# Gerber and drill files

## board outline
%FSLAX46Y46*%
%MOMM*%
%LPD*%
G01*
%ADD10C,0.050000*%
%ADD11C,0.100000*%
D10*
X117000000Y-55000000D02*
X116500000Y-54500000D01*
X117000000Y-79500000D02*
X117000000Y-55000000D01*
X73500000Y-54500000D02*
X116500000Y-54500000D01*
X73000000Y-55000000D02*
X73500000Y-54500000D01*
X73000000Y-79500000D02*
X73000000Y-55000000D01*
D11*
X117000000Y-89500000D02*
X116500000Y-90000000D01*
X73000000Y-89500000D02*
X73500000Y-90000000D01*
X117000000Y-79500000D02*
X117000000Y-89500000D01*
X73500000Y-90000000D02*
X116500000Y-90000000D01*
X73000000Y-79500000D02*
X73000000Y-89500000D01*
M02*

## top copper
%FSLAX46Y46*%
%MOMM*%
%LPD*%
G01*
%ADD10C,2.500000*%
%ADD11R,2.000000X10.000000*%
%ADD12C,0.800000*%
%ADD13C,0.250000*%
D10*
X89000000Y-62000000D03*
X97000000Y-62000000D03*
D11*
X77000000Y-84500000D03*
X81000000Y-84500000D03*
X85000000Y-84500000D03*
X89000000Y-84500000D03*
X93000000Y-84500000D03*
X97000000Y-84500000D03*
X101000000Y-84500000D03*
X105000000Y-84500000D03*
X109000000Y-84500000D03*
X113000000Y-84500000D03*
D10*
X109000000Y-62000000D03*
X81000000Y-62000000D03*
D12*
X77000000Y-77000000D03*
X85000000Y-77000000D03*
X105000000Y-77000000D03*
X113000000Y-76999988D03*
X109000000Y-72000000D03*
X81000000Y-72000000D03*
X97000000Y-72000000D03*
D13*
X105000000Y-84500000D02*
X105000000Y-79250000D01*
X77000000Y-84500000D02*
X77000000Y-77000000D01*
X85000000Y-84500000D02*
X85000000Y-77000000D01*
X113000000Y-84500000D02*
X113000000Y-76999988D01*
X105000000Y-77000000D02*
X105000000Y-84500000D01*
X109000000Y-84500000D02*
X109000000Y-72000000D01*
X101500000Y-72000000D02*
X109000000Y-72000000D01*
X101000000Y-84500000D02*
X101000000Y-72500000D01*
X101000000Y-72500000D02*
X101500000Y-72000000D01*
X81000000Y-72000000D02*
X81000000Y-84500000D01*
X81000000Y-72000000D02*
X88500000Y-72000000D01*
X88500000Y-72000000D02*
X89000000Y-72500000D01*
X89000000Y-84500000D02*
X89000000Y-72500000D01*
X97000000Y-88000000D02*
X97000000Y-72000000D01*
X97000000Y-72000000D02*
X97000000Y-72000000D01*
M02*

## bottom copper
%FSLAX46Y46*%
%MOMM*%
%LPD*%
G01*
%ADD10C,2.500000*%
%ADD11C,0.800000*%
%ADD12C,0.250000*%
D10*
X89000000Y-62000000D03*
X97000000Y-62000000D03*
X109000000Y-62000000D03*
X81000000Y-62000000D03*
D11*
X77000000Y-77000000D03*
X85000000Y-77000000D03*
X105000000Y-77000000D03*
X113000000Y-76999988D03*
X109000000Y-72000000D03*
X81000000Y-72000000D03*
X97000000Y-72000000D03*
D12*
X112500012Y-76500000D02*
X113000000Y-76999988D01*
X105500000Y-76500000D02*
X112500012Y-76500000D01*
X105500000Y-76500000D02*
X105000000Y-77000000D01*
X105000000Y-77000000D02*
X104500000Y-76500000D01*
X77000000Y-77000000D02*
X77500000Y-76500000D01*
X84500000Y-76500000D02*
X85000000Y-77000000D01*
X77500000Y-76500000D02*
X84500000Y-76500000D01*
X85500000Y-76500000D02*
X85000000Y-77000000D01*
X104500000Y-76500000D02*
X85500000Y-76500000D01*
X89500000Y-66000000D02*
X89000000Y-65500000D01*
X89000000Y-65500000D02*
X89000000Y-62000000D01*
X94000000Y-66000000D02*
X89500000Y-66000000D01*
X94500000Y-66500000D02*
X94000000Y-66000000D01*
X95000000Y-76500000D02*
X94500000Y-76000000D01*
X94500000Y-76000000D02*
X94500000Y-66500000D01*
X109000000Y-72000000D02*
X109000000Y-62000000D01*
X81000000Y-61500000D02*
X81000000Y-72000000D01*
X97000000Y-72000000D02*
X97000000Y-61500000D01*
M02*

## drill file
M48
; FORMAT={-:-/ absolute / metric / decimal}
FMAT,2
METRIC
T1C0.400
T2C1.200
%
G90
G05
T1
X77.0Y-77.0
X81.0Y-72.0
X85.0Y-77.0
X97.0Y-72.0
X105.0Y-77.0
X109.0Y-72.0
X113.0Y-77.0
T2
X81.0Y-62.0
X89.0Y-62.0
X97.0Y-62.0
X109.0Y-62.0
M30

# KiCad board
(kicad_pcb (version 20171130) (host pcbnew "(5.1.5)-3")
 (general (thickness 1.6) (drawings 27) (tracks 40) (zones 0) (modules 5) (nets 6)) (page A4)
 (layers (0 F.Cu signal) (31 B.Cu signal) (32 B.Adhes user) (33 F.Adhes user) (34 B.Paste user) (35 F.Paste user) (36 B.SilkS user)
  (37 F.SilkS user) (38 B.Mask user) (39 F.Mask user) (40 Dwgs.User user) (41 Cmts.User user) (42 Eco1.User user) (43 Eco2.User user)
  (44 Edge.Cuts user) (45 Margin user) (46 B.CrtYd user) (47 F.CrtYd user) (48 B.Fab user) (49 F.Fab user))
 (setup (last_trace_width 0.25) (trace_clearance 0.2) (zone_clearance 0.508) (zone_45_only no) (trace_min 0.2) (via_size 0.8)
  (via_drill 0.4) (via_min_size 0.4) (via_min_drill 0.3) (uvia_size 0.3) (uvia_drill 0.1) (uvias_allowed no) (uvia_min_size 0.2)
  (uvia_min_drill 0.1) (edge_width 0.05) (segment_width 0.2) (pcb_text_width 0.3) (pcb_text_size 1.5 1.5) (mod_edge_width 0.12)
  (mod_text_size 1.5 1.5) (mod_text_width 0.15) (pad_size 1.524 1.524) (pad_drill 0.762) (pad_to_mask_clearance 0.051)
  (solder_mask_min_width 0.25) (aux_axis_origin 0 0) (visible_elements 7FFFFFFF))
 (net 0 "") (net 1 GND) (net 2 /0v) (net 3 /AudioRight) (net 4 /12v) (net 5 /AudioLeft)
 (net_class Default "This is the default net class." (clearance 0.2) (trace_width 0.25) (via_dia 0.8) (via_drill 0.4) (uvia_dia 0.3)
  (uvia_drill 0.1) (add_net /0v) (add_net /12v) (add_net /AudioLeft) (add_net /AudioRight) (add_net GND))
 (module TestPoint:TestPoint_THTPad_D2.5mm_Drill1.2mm (layer F.Cu) (at 89 62)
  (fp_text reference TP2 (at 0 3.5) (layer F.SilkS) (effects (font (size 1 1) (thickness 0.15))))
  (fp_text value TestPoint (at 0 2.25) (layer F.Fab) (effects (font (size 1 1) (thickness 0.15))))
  (pad 1 thru_hole circle (at 0 0) (size 2.5 2.5) (drill 1.2) (layers *.Cu *.Mask) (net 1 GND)))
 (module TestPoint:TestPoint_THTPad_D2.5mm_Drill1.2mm (layer F.Cu) (at 97 62)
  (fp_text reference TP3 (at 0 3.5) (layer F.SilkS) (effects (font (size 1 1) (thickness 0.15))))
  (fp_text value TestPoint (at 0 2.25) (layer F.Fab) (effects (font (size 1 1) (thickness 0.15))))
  (pad 1 thru_hole circle (at 0 0) (size 2.5 2.5) (drill 1.2) (layers *.Cu *.Mask) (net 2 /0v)))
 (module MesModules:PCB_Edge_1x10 (layer F.Cu) (at 77 89.5)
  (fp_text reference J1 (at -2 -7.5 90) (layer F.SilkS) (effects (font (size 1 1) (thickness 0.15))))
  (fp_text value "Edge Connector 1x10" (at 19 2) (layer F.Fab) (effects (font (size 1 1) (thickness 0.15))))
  (fp_line (start 40 0) (end 39.5 0.5) (layer Edge.Cuts) (width 0.1))
  (fp_line (start -4 0) (end -3.5 0.5) (layer Edge.Cuts) (width 0.1))
  (fp_line (start 40 -10) (end 40 0) (layer Edge.Cuts) (width 0.1))
  (fp_line (start -3.5 0.5) (end 39.5 0.5) (layer Edge.Cuts) (width 0.1))
  (fp_line (start -4 -10) (end -4 0) (layer Edge.Cuts) (width 0.1))
  (pad 10 connect rect (at 0 -5) (size 2 10) (layers F.Cu F.Mask) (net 1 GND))
  (pad 9 connect rect (at 4 -5) (size 2 10) (layers F.Cu F.Mask) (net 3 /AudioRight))
  (pad 8 connect rect (at 8 -5) (size 2 10) (layers F.Cu F.Mask) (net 1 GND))
  (pad 7 connect rect (at 12 -5) (size 2 10) (layers F.Cu F.Mask) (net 3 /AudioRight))
  (pad 6 connect rect (at 16 -5) (size 2 10) (layers F.Cu F.Mask) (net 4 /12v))
  (pad 5 connect rect (at 20 -5) (size 2 10) (layers F.Cu F.Mask) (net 2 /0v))
  (pad 4 connect rect (at 24 -5) (size 2 10) (layers F.Cu F.Mask) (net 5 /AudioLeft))
  (pad 3 connect rect (at 28 -5) (size 2 10) (layers F.Cu F.Mask) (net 1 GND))
  (pad 2 connect rect (at 32 -5) (size 2 10) (layers F.Cu F.Mask) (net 5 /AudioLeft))
  (pad 1 connect rect (at 36 -5) (size 2 10) (layers F.Cu F.Mask) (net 1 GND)))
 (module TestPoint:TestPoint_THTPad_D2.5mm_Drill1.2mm (layer F.Cu) (at 109 62)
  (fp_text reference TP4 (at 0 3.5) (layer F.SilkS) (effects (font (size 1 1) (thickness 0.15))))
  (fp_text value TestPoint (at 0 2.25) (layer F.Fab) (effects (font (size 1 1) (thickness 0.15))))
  (pad 1 thru_hole circle (at 0 0) (size 2.5 2.5) (drill 1.2) (layers *.Cu *.Mask) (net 5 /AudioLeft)))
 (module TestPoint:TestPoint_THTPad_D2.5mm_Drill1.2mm (layer F.Cu) (at 81 62)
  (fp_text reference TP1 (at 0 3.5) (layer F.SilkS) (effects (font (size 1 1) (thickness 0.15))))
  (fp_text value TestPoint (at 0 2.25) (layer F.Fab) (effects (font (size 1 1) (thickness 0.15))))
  (pad 1 thru_hole circle (at 0 0) (size 2.5 2.5) (drill 1.2) (layers *.Cu *.Mask) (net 3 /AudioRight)))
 (gr_line (start 117 55) (end 116.5 54.5) (layer Edge.Cuts) (width 0.05))
 (gr_line (start 117 79.5) (end 117 55) (layer Edge.Cuts) (width 0.05))
 (gr_line (start 73.5 54.5) (end 116.5 54.5) (layer Edge.Cuts) (width 0.05))
 (gr_line (start 73 55) (end 73.5 54.5) (layer Edge.Cuts) (width 0.05))
 (gr_line (start 73 79.5) (end 73 55) (layer Edge.Cuts) (width 0.05))
 (via (at 77 77) (size 0.8) (drill 0.4) (layers F.Cu B.Cu) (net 1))
 (via (at 85 77) (size 0.8) (drill 0.4) (layers F.Cu B.Cu) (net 1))
 (via (at 105 77) (size 0.8) (drill 0.4) (layers F.Cu B.Cu) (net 1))
 (via (at 113 76.999988) (size 0.8) (drill 0.4) (layers F.Cu B.Cu) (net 1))
 (segment (start 105 84.5) (end 105 79.25) (width 0.25) (layer F.Cu) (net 1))
 (segment (start 112.500012 76.5) (end 113 76.999988) (width 0.25) (layer B.Cu) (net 1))
 (segment (start 105.5 76.5) (end 112.500012 76.5) (width 0.25) (layer B.Cu) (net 1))
 (segment (start 105.5 76.5) (end 105 77) (width 0.25) (layer B.Cu) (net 1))
 (segment (start 105 77) (end 104.5 76.5) (width 0.25) (layer B.Cu) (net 1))
 (segment (start 77 77) (end 77.5 76.5) (width 0.25) (layer B.Cu) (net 1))
 (segment (start 77 84.5) (end 77 77) (width 0.25) (layer F.Cu) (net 1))
 (segment (start 85 84.5) (end 85 77) (width 0.25) (layer F.Cu) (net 1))
 (segment (start 113 84.5) (end 113 76.999988) (width 0.25) (layer F.Cu) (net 1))
 (segment (start 105 77) (end 105 84.5) (width 0.25) (layer F.Cu) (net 1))
 (segment (start 84.5 76.5) (end 85 77) (width 0.25) (layer B.Cu) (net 1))
 (segment (start 77.5 76.5) (end 84.5 76.5) (width 0.25) (layer B.Cu) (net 1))
 (segment (start 85.5 76.5) (end 85 77) (width 0.25) (layer B.Cu) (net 1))
 (segment (start 104.5 76.5) (end 85.5 76.5) (width 0.25) (layer B.Cu) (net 1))
 (segment (start 89.5 66) (end 89 65.5) (width 0.25) (layer B.Cu) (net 1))
 (segment (start 89 65.5) (end 89 62) (width 0.25) (layer B.Cu) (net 1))
 (segment (start 94 66) (end 89.5 66) (width 0.25) (layer B.Cu) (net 1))
 (segment (start 94.5 66.5) (end 94 66) (width 0.25) (layer B.Cu) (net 1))
 (segment (start 95 76.5) (end 94.5 76) (width 0.25) (layer B.Cu) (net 1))
 (segment (start 94.5 76) (end 94.5 66.5) (width 0.25) (layer B.Cu) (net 1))
 (via (at 109 72) (size 0.8) (drill 0.4) (layers F.Cu B.Cu) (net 5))
 (segment (start 109 84.5) (end 109 72) (width 0.25) (layer F.Cu) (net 5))
 (segment (start 101.5 72) (end 109 72) (width 0.25) (layer F.Cu) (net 5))
 (segment (start 101 84.5) (end 101 72.5) (width 0.25) (layer F.Cu) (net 5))
 (segment (start 101 72.5) (end 101.5 72) (width 0.25) (layer F.Cu) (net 5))
 (segment (start 109 72) (end 109 62) (width 0.25) (layer B.Cu) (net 5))
 (segment (start 81 72) (end 81 84.5) (width 0.25) (layer F.Cu) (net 3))
 (via (at 81 72) (size 0.8) (drill 0.4) (layers F.Cu B.Cu) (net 3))
 (segment (start 81 72) (end 88.5 72) (width 0.25) (layer F.Cu) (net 3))
 (segment (start 88.5 72) (end 89 72.5) (width 0.25) (layer F.Cu) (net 3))
 (segment (start 89 84.5) (end 89 72.5) (width 0.25) (layer F.Cu) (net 3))
 (segment (start 81 61.5) (end 81 72) (width 0.25) (layer B.Cu) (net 3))
 (segment (start 97 88) (end 97 72) (width 0.25) (layer F.Cu) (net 2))
 (segment (start 97 72) (end 97 72) (width 0.25) (layer F.Cu) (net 2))
 (via (at 97 72) (size 0.8) (drill 0.4) (layers F.Cu B.Cu) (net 2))
 (segment (start 97 72) (end 97 61.5) (width 0.25) (layer B.Cu) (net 2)))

